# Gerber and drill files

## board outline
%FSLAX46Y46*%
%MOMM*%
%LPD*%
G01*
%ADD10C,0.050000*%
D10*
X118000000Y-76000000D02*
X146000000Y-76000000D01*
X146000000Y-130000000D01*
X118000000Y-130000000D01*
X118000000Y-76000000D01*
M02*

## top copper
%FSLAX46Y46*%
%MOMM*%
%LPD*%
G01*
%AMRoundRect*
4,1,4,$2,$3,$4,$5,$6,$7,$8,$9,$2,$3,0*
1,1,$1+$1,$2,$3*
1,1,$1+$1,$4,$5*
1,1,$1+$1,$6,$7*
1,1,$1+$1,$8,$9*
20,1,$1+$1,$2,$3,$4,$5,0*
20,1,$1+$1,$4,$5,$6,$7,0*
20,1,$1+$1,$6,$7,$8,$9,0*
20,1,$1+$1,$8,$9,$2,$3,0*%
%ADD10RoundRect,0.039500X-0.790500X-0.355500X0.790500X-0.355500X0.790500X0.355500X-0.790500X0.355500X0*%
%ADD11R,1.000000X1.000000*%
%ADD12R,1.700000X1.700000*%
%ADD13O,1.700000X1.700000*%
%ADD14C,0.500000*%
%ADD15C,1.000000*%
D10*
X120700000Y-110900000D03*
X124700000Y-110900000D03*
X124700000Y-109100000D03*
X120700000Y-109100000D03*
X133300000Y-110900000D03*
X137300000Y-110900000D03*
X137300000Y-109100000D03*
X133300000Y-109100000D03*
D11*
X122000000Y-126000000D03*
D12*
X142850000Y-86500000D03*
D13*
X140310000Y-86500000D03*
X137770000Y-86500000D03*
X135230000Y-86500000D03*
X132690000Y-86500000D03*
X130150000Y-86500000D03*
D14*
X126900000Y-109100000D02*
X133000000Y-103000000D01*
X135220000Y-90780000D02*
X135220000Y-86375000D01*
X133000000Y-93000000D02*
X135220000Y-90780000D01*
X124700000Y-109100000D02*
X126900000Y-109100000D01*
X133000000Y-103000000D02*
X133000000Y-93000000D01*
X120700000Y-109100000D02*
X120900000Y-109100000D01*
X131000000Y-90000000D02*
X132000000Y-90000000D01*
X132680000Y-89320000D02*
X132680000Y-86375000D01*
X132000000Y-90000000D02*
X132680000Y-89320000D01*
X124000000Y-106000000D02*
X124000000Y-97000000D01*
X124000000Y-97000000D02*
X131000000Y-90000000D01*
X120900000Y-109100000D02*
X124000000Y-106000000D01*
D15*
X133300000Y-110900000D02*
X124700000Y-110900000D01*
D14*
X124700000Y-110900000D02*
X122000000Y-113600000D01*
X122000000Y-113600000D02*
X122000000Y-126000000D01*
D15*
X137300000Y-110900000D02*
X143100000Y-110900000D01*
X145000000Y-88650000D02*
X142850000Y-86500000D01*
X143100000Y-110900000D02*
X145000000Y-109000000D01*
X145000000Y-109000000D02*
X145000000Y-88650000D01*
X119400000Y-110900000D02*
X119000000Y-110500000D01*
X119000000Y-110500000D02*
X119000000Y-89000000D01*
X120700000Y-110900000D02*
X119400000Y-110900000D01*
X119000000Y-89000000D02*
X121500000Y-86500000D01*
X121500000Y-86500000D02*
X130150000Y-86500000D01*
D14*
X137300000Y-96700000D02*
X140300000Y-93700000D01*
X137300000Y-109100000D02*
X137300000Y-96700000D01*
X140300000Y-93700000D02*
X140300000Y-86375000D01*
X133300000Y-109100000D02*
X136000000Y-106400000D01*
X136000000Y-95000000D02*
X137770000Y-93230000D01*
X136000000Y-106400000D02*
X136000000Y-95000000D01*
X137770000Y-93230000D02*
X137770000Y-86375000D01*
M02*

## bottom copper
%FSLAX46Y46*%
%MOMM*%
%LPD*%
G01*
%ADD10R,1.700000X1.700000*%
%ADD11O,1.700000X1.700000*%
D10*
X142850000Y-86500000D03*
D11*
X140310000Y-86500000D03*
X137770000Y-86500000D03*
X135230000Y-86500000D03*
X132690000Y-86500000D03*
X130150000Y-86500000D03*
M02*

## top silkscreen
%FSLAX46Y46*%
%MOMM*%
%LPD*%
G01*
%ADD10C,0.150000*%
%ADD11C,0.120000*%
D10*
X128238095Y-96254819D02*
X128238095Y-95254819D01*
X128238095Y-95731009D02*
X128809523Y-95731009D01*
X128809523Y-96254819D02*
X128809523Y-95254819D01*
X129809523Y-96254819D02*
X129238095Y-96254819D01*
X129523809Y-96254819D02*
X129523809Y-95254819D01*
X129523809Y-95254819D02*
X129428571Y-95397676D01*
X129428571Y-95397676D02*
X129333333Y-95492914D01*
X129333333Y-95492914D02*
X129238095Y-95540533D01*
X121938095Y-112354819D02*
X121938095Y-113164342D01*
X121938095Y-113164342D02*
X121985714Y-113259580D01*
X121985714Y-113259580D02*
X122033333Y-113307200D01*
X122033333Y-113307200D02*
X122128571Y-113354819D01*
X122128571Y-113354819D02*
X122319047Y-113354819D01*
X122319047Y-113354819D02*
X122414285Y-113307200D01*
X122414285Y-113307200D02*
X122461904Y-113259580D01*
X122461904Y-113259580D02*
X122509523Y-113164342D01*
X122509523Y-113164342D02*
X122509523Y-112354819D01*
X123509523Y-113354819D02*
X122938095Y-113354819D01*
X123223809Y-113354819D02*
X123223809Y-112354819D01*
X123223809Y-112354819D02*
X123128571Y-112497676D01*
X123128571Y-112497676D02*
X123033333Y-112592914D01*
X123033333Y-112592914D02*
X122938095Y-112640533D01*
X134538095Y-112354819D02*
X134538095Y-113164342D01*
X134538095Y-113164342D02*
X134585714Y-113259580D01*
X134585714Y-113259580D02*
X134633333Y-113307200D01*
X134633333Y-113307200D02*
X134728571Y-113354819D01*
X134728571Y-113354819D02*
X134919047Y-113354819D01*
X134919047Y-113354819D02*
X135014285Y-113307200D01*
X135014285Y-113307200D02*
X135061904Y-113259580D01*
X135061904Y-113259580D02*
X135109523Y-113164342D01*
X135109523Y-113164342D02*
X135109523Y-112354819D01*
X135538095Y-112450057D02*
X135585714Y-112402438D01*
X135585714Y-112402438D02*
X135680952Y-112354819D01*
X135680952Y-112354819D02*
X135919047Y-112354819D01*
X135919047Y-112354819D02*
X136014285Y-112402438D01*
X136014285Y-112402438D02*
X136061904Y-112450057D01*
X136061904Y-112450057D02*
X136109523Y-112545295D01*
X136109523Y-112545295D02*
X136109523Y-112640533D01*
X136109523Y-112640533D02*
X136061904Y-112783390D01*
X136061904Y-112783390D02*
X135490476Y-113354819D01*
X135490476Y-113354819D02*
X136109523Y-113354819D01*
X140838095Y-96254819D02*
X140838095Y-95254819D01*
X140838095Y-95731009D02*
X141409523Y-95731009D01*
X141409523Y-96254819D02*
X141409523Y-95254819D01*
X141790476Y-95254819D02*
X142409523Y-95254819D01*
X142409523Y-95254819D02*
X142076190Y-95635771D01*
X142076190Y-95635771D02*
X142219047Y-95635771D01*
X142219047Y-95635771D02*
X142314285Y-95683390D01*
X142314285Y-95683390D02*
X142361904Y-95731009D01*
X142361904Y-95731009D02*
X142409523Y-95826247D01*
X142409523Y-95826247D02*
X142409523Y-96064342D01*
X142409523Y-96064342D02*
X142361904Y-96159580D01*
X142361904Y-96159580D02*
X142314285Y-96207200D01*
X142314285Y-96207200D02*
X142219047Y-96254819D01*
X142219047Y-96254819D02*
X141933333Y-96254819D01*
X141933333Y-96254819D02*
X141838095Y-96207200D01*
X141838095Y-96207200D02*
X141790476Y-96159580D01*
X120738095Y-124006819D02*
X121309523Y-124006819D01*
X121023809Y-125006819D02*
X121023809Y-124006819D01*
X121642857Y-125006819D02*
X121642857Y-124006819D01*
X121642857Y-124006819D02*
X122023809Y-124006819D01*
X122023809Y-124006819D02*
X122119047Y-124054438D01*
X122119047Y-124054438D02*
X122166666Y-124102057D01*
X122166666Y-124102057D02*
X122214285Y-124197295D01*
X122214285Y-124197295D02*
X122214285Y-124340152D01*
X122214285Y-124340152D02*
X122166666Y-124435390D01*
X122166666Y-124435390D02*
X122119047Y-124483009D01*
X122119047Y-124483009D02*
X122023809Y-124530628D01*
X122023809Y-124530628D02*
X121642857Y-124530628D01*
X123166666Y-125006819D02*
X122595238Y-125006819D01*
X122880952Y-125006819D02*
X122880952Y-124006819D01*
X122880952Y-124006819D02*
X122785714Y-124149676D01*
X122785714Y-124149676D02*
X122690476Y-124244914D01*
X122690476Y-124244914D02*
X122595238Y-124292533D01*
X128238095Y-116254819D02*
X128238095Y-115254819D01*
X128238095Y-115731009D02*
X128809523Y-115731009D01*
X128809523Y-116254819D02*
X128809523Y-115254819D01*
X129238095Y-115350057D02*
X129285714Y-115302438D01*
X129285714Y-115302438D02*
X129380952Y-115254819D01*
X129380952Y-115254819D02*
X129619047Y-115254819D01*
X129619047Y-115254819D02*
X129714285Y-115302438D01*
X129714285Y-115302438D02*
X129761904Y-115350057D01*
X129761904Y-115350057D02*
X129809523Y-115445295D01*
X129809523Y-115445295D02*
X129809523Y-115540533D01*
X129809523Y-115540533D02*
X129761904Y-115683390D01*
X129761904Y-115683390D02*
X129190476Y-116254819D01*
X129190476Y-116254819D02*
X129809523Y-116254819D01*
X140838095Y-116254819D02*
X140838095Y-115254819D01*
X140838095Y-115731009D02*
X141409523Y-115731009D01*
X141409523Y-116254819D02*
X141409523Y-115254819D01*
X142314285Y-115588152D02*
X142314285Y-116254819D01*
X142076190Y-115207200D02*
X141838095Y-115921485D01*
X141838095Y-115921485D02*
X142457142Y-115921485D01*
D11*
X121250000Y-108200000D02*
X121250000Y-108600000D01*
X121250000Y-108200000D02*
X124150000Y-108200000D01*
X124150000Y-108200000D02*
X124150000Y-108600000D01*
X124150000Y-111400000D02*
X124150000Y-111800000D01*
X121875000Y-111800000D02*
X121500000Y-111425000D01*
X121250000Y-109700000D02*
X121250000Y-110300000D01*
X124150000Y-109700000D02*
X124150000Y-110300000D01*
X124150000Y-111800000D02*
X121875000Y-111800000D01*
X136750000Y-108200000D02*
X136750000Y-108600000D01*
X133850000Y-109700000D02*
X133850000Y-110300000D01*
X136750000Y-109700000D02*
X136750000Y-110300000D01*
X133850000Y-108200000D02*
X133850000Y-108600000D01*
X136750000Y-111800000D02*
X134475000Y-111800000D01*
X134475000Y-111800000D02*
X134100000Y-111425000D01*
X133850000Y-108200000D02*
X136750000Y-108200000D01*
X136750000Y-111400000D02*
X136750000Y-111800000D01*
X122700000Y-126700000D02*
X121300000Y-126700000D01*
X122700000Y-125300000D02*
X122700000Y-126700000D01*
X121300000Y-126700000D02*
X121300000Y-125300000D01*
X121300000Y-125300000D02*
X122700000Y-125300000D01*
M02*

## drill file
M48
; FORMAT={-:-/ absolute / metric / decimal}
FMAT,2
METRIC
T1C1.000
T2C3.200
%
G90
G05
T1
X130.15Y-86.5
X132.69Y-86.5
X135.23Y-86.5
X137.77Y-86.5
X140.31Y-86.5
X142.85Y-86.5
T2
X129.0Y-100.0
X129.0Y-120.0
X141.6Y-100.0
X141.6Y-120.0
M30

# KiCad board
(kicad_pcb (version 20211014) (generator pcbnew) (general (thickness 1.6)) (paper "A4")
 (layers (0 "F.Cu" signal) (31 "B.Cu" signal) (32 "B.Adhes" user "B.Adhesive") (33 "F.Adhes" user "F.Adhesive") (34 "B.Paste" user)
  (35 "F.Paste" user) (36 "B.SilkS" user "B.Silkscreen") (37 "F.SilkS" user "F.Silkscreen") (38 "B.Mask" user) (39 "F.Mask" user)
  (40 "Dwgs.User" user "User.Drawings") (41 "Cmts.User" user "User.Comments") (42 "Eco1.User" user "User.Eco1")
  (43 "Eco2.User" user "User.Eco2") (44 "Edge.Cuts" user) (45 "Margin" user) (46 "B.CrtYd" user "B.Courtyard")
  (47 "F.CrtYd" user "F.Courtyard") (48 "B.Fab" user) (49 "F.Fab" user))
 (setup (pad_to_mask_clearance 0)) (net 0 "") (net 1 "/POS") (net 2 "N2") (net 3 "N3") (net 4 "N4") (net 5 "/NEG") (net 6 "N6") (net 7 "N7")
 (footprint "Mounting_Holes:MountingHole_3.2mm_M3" (layer "F.Cu") (at 129 100)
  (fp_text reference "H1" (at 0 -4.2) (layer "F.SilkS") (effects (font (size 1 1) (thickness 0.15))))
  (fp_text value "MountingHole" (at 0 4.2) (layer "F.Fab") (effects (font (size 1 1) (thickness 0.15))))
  (pad "" np_thru_hole circle (at 0 0) (size 3.2 3.2) (drill 3.2) (layers *.Cu *.Mask)))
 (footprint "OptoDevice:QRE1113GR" (layer "F.Cu") (at 122.7 110)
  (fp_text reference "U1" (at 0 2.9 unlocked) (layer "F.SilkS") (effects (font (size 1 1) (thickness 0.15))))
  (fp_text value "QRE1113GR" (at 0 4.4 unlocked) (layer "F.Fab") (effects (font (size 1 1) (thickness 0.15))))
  (fp_line (start -1.45 -1.8) (end -1.45 -1.4) (layer "F.SilkS") (width 0.12))
  (fp_line (start -1.45 -1.8) (end 1.45 -1.8) (layer "F.SilkS") (width 0.12))
  (fp_line (start 1.45 -1.8) (end 1.45 -1.4) (layer "F.SilkS") (width 0.12))
  (fp_line (start 1.45 1.4) (end 1.45 1.8) (layer "F.SilkS") (width 0.12))
  (fp_line (start -0.825 1.8) (end -1.2 1.425) (layer "F.SilkS") (width 0.12))
  (fp_line (start -1.45 -0.3) (end -1.45 0.3) (layer "F.SilkS") (width 0.12))
  (fp_line (start 1.45 -0.3) (end 1.45 0.3) (layer "F.SilkS") (width 0.12))
  (fp_line (start 1.45 1.8) (end -0.825 1.8) (layer "F.SilkS") (width 0.12))
  (pad "1" smd roundrect (at -2 0.9) (size 1.66 0.79) (layers "F.Cu" "F.Paste" "F.Mask") (roundrect_rratio 0.05) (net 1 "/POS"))
  (pad "2" smd roundrect (at 2 0.9) (size 1.66 0.79) (layers "F.Cu" "F.Paste" "F.Mask") (roundrect_rratio 0.05) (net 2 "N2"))
  (pad "3" smd roundrect (at 2 -0.9) (size 1.66 0.79) (layers "F.Cu" "F.Paste" "F.Mask") (roundrect_rratio 0.05) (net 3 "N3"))
  (pad "4" smd roundrect (at -2 -0.9) (size 1.66 0.79) (layers "F.Cu" "F.Paste" "F.Mask") (roundrect_rratio 0.05) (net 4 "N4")))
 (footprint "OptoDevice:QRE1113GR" (layer "F.Cu") (at 135.3 110)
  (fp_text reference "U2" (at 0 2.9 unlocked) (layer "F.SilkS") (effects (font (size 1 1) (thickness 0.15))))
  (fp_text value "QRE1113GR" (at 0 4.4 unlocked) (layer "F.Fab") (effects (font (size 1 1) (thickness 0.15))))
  (fp_line (start 1.45 -1.8) (end 1.45 -1.4) (layer "F.SilkS") (width 0.12))
  (fp_line (start -1.45 -0.3) (end -1.45 0.3) (layer "F.SilkS") (width 0.12))
  (fp_line (start 1.45 -0.3) (end 1.45 0.3) (layer "F.SilkS") (width 0.12))
  (fp_line (start -1.45 -1.8) (end -1.45 -1.4) (layer "F.SilkS") (width 0.12))
  (fp_line (start 1.45 1.8) (end -0.825 1.8) (layer "F.SilkS") (width 0.12))
  (fp_line (start -0.825 1.8) (end -1.2 1.425) (layer "F.SilkS") (width 0.12))
  (fp_line (start -1.45 -1.8) (end 1.45 -1.8) (layer "F.SilkS") (width 0.12))
  (fp_line (start 1.45 1.4) (end 1.45 1.8) (layer "F.SilkS") (width 0.12))
  (pad "1" smd roundrect (at -2 0.9) (size 1.66 0.79) (layers "F.Cu" "F.Paste" "F.Mask") (roundrect_rratio 0.05) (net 2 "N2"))
  (pad "2" smd roundrect (at 2 0.9) (size 1.66 0.79) (layers "F.Cu" "F.Paste" "F.Mask") (roundrect_rratio 0.05) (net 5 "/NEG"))
  (pad "3" smd roundrect (at 2 -0.9) (size 1.66 0.79) (layers "F.Cu" "F.Paste" "F.Mask") (roundrect_rratio 0.05) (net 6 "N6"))
  (pad "4" smd roundrect (at -2 -0.9) (size 1.66 0.79) (layers "F.Cu" "F.Paste" "F.Mask") (roundrect_rratio 0.05) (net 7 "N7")))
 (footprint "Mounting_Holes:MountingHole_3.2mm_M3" (layer "F.Cu") (at 141.6 100)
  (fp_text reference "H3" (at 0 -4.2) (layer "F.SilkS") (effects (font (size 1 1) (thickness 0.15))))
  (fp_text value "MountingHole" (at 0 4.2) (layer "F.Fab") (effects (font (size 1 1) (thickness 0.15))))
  (pad "" np_thru_hole circle (at 0 0) (size 3.2 3.2) (drill 3.2) (layers *.Cu *.Mask)))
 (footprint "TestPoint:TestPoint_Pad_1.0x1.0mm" (layer "F.Cu") (at 122 126)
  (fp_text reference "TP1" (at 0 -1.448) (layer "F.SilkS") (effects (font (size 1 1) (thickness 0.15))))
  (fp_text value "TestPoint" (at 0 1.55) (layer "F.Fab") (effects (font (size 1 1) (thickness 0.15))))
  (fp_line (start 0.7 0.7) (end -0.7 0.7) (layer "F.SilkS") (width 0.12))
  (fp_line (start 0.7 -0.7) (end 0.7 0.7) (layer "F.SilkS") (width 0.12))
  (fp_line (start -0.7 0.7) (end -0.7 -0.7) (layer "F.SilkS") (width 0.12))
  (fp_line (start -0.7 -0.7) (end 0.7 -0.7) (layer "F.SilkS") (width 0.12))
  (pad "1" smd rect locked (at 0 0) (size 1 1) (layers "F.Cu" "F.Mask") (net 2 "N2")))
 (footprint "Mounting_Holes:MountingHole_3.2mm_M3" (layer "F.Cu") (at 129 120)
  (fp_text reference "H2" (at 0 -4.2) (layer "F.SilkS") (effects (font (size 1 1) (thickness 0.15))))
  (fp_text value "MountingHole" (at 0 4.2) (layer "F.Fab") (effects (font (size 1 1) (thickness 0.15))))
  (pad "" np_thru_hole circle (at 0 0) (size 3.2 3.2) (drill 3.2) (layers *.Cu *.Mask)))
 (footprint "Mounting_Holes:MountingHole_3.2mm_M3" (layer "F.Cu") (at 141.6 120)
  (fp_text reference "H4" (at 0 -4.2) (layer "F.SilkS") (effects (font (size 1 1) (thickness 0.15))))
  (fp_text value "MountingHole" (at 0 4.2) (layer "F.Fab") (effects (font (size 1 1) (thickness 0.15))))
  (pad "" np_thru_hole circle (at 0 0) (size 3.2 3.2) (drill 3.2) (layers *.Cu *.Mask)))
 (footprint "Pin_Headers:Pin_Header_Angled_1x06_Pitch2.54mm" (layer "B.Cu") (at 142.85 86.5 90)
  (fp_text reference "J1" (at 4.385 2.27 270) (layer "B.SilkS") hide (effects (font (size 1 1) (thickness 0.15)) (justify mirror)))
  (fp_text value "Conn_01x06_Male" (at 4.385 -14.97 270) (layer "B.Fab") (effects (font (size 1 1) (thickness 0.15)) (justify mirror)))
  (pad "1" thru_hole rect (at 0 0 90) (size 1.7 1.7) (drill 1) (layers *.Cu *.Mask) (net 5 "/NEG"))
  (pad "2" thru_hole oval (at 0 -2.54 90) (size 1.7 1.7) (drill 1) (layers *.Cu *.Mask) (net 6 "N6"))
  (pad "3" thru_hole oval (at 0 -5.08 90) (size 1.7 1.7) (drill 1) (layers *.Cu *.Mask) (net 7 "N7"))
  (pad "4" thru_hole oval (at 0 -7.62 90) (size 1.7 1.7) (drill 1) (layers *.Cu *.Mask) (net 3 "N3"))
  (pad "5" thru_hole oval (at 0 -10.16 90) (size 1.7 1.7) (drill 1) (layers *.Cu *.Mask) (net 4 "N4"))
  (pad "6" thru_hole oval (at 0 -12.7 90) (size 1.7 1.7) (drill 1) (layers *.Cu *.Mask) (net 1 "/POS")))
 (gr_rect (start 118 76) (end 146 130) (layer "Edge.Cuts") (width 0.05) (fill none))
 (segment (start 126.9 109.1) (end 133 103) (width 0.5) (layer "F.Cu") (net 3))
 (segment (start 135.22 90.78) (end 135.22 86.375) (width 0.5) (layer "F.Cu") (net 3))
 (segment (start 133 93) (end 135.22 90.78) (width 0.5) (layer "F.Cu") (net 3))
 (segment (start 124.7 109.1) (end 126.9 109.1) (width 0.5) (layer "F.Cu") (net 3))
 (segment (start 133 103) (end 133 93) (width 0.5) (layer "F.Cu") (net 3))
 (segment (start 120.7 109.1) (end 120.9 109.1) (width 0.5) (layer "F.Cu") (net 4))
 (segment (start 131 90) (end 132 90) (width 0.5) (layer "F.Cu") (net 4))
 (segment (start 132.68 89.32) (end 132.68 86.375) (width 0.5) (layer "F.Cu") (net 4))
 (segment (start 132 90) (end 132.68 89.32) (width 0.5) (layer "F.Cu") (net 4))
 (segment (start 124 106) (end 124 97) (width 0.5) (layer "F.Cu") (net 4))
 (segment (start 124 97) (end 131 90) (width 0.5) (layer "F.Cu") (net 4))
 (segment (start 120.9 109.1) (end 124 106) (width 0.5) (layer "F.Cu") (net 4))
 (segment (start 133.3 110.9) (end 124.7 110.9) (width 1) (layer "F.Cu") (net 2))
 (segment (start 124.7 110.9) (end 122 113.6) (width 0.5) (layer "F.Cu") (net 2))
 (segment (start 122 113.6) (end 122 126) (width 0.5) (layer "F.Cu") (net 2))
 (segment (start 137.3 110.9) (end 143.1 110.9) (width 1) (layer "F.Cu") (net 5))
 (segment (start 145 88.65) (end 142.85 86.5) (width 1) (layer "F.Cu") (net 5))
 (segment (start 143.1 110.9) (end 145 109) (width 1) (layer "F.Cu") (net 5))
 (segment (start 145 109) (end 145 88.65) (width 1) (layer "F.Cu") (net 5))
 (segment (start 119.4 110.9) (end 119 110.5) (width 1) (layer "F.Cu") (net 1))
 (segment (start 119 110.5) (end 119 89) (width 1) (layer "F.Cu") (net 1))
 (segment (start 120.7 110.9) (end 119.4 110.9) (width 1) (layer "F.Cu") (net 1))
 (segment (start 119 89) (end 121.5 86.5) (width 1) (layer "F.Cu") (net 1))
 (segment (start 121.5 86.5) (end 130.15 86.5) (width 1) (layer "F.Cu") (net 1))
 (segment (start 137.3 96.7) (end 140.3 93.7) (width 0.5) (layer "F.Cu") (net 6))
 (segment (start 137.3 109.1) (end 137.3 96.7) (width 0.5) (layer "F.Cu") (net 6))
 (segment (start 140.3 93.7) (end 140.3 86.375) (width 0.5) (layer "F.Cu") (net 6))
 (segment (start 133.3 109.1) (end 136 106.4) (width 0.5) (layer "F.Cu") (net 7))
 (segment (start 136 95) (end 137.77 93.23) (width 0.5) (layer "F.Cu") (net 7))
 (segment (start 136 106.4) (end 136 95) (width 0.5) (layer "F.Cu") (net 7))
 (segment (start 137.77 93.23) (end 137.77 86.375) (width 0.5) (layer "F.Cu") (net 7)))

